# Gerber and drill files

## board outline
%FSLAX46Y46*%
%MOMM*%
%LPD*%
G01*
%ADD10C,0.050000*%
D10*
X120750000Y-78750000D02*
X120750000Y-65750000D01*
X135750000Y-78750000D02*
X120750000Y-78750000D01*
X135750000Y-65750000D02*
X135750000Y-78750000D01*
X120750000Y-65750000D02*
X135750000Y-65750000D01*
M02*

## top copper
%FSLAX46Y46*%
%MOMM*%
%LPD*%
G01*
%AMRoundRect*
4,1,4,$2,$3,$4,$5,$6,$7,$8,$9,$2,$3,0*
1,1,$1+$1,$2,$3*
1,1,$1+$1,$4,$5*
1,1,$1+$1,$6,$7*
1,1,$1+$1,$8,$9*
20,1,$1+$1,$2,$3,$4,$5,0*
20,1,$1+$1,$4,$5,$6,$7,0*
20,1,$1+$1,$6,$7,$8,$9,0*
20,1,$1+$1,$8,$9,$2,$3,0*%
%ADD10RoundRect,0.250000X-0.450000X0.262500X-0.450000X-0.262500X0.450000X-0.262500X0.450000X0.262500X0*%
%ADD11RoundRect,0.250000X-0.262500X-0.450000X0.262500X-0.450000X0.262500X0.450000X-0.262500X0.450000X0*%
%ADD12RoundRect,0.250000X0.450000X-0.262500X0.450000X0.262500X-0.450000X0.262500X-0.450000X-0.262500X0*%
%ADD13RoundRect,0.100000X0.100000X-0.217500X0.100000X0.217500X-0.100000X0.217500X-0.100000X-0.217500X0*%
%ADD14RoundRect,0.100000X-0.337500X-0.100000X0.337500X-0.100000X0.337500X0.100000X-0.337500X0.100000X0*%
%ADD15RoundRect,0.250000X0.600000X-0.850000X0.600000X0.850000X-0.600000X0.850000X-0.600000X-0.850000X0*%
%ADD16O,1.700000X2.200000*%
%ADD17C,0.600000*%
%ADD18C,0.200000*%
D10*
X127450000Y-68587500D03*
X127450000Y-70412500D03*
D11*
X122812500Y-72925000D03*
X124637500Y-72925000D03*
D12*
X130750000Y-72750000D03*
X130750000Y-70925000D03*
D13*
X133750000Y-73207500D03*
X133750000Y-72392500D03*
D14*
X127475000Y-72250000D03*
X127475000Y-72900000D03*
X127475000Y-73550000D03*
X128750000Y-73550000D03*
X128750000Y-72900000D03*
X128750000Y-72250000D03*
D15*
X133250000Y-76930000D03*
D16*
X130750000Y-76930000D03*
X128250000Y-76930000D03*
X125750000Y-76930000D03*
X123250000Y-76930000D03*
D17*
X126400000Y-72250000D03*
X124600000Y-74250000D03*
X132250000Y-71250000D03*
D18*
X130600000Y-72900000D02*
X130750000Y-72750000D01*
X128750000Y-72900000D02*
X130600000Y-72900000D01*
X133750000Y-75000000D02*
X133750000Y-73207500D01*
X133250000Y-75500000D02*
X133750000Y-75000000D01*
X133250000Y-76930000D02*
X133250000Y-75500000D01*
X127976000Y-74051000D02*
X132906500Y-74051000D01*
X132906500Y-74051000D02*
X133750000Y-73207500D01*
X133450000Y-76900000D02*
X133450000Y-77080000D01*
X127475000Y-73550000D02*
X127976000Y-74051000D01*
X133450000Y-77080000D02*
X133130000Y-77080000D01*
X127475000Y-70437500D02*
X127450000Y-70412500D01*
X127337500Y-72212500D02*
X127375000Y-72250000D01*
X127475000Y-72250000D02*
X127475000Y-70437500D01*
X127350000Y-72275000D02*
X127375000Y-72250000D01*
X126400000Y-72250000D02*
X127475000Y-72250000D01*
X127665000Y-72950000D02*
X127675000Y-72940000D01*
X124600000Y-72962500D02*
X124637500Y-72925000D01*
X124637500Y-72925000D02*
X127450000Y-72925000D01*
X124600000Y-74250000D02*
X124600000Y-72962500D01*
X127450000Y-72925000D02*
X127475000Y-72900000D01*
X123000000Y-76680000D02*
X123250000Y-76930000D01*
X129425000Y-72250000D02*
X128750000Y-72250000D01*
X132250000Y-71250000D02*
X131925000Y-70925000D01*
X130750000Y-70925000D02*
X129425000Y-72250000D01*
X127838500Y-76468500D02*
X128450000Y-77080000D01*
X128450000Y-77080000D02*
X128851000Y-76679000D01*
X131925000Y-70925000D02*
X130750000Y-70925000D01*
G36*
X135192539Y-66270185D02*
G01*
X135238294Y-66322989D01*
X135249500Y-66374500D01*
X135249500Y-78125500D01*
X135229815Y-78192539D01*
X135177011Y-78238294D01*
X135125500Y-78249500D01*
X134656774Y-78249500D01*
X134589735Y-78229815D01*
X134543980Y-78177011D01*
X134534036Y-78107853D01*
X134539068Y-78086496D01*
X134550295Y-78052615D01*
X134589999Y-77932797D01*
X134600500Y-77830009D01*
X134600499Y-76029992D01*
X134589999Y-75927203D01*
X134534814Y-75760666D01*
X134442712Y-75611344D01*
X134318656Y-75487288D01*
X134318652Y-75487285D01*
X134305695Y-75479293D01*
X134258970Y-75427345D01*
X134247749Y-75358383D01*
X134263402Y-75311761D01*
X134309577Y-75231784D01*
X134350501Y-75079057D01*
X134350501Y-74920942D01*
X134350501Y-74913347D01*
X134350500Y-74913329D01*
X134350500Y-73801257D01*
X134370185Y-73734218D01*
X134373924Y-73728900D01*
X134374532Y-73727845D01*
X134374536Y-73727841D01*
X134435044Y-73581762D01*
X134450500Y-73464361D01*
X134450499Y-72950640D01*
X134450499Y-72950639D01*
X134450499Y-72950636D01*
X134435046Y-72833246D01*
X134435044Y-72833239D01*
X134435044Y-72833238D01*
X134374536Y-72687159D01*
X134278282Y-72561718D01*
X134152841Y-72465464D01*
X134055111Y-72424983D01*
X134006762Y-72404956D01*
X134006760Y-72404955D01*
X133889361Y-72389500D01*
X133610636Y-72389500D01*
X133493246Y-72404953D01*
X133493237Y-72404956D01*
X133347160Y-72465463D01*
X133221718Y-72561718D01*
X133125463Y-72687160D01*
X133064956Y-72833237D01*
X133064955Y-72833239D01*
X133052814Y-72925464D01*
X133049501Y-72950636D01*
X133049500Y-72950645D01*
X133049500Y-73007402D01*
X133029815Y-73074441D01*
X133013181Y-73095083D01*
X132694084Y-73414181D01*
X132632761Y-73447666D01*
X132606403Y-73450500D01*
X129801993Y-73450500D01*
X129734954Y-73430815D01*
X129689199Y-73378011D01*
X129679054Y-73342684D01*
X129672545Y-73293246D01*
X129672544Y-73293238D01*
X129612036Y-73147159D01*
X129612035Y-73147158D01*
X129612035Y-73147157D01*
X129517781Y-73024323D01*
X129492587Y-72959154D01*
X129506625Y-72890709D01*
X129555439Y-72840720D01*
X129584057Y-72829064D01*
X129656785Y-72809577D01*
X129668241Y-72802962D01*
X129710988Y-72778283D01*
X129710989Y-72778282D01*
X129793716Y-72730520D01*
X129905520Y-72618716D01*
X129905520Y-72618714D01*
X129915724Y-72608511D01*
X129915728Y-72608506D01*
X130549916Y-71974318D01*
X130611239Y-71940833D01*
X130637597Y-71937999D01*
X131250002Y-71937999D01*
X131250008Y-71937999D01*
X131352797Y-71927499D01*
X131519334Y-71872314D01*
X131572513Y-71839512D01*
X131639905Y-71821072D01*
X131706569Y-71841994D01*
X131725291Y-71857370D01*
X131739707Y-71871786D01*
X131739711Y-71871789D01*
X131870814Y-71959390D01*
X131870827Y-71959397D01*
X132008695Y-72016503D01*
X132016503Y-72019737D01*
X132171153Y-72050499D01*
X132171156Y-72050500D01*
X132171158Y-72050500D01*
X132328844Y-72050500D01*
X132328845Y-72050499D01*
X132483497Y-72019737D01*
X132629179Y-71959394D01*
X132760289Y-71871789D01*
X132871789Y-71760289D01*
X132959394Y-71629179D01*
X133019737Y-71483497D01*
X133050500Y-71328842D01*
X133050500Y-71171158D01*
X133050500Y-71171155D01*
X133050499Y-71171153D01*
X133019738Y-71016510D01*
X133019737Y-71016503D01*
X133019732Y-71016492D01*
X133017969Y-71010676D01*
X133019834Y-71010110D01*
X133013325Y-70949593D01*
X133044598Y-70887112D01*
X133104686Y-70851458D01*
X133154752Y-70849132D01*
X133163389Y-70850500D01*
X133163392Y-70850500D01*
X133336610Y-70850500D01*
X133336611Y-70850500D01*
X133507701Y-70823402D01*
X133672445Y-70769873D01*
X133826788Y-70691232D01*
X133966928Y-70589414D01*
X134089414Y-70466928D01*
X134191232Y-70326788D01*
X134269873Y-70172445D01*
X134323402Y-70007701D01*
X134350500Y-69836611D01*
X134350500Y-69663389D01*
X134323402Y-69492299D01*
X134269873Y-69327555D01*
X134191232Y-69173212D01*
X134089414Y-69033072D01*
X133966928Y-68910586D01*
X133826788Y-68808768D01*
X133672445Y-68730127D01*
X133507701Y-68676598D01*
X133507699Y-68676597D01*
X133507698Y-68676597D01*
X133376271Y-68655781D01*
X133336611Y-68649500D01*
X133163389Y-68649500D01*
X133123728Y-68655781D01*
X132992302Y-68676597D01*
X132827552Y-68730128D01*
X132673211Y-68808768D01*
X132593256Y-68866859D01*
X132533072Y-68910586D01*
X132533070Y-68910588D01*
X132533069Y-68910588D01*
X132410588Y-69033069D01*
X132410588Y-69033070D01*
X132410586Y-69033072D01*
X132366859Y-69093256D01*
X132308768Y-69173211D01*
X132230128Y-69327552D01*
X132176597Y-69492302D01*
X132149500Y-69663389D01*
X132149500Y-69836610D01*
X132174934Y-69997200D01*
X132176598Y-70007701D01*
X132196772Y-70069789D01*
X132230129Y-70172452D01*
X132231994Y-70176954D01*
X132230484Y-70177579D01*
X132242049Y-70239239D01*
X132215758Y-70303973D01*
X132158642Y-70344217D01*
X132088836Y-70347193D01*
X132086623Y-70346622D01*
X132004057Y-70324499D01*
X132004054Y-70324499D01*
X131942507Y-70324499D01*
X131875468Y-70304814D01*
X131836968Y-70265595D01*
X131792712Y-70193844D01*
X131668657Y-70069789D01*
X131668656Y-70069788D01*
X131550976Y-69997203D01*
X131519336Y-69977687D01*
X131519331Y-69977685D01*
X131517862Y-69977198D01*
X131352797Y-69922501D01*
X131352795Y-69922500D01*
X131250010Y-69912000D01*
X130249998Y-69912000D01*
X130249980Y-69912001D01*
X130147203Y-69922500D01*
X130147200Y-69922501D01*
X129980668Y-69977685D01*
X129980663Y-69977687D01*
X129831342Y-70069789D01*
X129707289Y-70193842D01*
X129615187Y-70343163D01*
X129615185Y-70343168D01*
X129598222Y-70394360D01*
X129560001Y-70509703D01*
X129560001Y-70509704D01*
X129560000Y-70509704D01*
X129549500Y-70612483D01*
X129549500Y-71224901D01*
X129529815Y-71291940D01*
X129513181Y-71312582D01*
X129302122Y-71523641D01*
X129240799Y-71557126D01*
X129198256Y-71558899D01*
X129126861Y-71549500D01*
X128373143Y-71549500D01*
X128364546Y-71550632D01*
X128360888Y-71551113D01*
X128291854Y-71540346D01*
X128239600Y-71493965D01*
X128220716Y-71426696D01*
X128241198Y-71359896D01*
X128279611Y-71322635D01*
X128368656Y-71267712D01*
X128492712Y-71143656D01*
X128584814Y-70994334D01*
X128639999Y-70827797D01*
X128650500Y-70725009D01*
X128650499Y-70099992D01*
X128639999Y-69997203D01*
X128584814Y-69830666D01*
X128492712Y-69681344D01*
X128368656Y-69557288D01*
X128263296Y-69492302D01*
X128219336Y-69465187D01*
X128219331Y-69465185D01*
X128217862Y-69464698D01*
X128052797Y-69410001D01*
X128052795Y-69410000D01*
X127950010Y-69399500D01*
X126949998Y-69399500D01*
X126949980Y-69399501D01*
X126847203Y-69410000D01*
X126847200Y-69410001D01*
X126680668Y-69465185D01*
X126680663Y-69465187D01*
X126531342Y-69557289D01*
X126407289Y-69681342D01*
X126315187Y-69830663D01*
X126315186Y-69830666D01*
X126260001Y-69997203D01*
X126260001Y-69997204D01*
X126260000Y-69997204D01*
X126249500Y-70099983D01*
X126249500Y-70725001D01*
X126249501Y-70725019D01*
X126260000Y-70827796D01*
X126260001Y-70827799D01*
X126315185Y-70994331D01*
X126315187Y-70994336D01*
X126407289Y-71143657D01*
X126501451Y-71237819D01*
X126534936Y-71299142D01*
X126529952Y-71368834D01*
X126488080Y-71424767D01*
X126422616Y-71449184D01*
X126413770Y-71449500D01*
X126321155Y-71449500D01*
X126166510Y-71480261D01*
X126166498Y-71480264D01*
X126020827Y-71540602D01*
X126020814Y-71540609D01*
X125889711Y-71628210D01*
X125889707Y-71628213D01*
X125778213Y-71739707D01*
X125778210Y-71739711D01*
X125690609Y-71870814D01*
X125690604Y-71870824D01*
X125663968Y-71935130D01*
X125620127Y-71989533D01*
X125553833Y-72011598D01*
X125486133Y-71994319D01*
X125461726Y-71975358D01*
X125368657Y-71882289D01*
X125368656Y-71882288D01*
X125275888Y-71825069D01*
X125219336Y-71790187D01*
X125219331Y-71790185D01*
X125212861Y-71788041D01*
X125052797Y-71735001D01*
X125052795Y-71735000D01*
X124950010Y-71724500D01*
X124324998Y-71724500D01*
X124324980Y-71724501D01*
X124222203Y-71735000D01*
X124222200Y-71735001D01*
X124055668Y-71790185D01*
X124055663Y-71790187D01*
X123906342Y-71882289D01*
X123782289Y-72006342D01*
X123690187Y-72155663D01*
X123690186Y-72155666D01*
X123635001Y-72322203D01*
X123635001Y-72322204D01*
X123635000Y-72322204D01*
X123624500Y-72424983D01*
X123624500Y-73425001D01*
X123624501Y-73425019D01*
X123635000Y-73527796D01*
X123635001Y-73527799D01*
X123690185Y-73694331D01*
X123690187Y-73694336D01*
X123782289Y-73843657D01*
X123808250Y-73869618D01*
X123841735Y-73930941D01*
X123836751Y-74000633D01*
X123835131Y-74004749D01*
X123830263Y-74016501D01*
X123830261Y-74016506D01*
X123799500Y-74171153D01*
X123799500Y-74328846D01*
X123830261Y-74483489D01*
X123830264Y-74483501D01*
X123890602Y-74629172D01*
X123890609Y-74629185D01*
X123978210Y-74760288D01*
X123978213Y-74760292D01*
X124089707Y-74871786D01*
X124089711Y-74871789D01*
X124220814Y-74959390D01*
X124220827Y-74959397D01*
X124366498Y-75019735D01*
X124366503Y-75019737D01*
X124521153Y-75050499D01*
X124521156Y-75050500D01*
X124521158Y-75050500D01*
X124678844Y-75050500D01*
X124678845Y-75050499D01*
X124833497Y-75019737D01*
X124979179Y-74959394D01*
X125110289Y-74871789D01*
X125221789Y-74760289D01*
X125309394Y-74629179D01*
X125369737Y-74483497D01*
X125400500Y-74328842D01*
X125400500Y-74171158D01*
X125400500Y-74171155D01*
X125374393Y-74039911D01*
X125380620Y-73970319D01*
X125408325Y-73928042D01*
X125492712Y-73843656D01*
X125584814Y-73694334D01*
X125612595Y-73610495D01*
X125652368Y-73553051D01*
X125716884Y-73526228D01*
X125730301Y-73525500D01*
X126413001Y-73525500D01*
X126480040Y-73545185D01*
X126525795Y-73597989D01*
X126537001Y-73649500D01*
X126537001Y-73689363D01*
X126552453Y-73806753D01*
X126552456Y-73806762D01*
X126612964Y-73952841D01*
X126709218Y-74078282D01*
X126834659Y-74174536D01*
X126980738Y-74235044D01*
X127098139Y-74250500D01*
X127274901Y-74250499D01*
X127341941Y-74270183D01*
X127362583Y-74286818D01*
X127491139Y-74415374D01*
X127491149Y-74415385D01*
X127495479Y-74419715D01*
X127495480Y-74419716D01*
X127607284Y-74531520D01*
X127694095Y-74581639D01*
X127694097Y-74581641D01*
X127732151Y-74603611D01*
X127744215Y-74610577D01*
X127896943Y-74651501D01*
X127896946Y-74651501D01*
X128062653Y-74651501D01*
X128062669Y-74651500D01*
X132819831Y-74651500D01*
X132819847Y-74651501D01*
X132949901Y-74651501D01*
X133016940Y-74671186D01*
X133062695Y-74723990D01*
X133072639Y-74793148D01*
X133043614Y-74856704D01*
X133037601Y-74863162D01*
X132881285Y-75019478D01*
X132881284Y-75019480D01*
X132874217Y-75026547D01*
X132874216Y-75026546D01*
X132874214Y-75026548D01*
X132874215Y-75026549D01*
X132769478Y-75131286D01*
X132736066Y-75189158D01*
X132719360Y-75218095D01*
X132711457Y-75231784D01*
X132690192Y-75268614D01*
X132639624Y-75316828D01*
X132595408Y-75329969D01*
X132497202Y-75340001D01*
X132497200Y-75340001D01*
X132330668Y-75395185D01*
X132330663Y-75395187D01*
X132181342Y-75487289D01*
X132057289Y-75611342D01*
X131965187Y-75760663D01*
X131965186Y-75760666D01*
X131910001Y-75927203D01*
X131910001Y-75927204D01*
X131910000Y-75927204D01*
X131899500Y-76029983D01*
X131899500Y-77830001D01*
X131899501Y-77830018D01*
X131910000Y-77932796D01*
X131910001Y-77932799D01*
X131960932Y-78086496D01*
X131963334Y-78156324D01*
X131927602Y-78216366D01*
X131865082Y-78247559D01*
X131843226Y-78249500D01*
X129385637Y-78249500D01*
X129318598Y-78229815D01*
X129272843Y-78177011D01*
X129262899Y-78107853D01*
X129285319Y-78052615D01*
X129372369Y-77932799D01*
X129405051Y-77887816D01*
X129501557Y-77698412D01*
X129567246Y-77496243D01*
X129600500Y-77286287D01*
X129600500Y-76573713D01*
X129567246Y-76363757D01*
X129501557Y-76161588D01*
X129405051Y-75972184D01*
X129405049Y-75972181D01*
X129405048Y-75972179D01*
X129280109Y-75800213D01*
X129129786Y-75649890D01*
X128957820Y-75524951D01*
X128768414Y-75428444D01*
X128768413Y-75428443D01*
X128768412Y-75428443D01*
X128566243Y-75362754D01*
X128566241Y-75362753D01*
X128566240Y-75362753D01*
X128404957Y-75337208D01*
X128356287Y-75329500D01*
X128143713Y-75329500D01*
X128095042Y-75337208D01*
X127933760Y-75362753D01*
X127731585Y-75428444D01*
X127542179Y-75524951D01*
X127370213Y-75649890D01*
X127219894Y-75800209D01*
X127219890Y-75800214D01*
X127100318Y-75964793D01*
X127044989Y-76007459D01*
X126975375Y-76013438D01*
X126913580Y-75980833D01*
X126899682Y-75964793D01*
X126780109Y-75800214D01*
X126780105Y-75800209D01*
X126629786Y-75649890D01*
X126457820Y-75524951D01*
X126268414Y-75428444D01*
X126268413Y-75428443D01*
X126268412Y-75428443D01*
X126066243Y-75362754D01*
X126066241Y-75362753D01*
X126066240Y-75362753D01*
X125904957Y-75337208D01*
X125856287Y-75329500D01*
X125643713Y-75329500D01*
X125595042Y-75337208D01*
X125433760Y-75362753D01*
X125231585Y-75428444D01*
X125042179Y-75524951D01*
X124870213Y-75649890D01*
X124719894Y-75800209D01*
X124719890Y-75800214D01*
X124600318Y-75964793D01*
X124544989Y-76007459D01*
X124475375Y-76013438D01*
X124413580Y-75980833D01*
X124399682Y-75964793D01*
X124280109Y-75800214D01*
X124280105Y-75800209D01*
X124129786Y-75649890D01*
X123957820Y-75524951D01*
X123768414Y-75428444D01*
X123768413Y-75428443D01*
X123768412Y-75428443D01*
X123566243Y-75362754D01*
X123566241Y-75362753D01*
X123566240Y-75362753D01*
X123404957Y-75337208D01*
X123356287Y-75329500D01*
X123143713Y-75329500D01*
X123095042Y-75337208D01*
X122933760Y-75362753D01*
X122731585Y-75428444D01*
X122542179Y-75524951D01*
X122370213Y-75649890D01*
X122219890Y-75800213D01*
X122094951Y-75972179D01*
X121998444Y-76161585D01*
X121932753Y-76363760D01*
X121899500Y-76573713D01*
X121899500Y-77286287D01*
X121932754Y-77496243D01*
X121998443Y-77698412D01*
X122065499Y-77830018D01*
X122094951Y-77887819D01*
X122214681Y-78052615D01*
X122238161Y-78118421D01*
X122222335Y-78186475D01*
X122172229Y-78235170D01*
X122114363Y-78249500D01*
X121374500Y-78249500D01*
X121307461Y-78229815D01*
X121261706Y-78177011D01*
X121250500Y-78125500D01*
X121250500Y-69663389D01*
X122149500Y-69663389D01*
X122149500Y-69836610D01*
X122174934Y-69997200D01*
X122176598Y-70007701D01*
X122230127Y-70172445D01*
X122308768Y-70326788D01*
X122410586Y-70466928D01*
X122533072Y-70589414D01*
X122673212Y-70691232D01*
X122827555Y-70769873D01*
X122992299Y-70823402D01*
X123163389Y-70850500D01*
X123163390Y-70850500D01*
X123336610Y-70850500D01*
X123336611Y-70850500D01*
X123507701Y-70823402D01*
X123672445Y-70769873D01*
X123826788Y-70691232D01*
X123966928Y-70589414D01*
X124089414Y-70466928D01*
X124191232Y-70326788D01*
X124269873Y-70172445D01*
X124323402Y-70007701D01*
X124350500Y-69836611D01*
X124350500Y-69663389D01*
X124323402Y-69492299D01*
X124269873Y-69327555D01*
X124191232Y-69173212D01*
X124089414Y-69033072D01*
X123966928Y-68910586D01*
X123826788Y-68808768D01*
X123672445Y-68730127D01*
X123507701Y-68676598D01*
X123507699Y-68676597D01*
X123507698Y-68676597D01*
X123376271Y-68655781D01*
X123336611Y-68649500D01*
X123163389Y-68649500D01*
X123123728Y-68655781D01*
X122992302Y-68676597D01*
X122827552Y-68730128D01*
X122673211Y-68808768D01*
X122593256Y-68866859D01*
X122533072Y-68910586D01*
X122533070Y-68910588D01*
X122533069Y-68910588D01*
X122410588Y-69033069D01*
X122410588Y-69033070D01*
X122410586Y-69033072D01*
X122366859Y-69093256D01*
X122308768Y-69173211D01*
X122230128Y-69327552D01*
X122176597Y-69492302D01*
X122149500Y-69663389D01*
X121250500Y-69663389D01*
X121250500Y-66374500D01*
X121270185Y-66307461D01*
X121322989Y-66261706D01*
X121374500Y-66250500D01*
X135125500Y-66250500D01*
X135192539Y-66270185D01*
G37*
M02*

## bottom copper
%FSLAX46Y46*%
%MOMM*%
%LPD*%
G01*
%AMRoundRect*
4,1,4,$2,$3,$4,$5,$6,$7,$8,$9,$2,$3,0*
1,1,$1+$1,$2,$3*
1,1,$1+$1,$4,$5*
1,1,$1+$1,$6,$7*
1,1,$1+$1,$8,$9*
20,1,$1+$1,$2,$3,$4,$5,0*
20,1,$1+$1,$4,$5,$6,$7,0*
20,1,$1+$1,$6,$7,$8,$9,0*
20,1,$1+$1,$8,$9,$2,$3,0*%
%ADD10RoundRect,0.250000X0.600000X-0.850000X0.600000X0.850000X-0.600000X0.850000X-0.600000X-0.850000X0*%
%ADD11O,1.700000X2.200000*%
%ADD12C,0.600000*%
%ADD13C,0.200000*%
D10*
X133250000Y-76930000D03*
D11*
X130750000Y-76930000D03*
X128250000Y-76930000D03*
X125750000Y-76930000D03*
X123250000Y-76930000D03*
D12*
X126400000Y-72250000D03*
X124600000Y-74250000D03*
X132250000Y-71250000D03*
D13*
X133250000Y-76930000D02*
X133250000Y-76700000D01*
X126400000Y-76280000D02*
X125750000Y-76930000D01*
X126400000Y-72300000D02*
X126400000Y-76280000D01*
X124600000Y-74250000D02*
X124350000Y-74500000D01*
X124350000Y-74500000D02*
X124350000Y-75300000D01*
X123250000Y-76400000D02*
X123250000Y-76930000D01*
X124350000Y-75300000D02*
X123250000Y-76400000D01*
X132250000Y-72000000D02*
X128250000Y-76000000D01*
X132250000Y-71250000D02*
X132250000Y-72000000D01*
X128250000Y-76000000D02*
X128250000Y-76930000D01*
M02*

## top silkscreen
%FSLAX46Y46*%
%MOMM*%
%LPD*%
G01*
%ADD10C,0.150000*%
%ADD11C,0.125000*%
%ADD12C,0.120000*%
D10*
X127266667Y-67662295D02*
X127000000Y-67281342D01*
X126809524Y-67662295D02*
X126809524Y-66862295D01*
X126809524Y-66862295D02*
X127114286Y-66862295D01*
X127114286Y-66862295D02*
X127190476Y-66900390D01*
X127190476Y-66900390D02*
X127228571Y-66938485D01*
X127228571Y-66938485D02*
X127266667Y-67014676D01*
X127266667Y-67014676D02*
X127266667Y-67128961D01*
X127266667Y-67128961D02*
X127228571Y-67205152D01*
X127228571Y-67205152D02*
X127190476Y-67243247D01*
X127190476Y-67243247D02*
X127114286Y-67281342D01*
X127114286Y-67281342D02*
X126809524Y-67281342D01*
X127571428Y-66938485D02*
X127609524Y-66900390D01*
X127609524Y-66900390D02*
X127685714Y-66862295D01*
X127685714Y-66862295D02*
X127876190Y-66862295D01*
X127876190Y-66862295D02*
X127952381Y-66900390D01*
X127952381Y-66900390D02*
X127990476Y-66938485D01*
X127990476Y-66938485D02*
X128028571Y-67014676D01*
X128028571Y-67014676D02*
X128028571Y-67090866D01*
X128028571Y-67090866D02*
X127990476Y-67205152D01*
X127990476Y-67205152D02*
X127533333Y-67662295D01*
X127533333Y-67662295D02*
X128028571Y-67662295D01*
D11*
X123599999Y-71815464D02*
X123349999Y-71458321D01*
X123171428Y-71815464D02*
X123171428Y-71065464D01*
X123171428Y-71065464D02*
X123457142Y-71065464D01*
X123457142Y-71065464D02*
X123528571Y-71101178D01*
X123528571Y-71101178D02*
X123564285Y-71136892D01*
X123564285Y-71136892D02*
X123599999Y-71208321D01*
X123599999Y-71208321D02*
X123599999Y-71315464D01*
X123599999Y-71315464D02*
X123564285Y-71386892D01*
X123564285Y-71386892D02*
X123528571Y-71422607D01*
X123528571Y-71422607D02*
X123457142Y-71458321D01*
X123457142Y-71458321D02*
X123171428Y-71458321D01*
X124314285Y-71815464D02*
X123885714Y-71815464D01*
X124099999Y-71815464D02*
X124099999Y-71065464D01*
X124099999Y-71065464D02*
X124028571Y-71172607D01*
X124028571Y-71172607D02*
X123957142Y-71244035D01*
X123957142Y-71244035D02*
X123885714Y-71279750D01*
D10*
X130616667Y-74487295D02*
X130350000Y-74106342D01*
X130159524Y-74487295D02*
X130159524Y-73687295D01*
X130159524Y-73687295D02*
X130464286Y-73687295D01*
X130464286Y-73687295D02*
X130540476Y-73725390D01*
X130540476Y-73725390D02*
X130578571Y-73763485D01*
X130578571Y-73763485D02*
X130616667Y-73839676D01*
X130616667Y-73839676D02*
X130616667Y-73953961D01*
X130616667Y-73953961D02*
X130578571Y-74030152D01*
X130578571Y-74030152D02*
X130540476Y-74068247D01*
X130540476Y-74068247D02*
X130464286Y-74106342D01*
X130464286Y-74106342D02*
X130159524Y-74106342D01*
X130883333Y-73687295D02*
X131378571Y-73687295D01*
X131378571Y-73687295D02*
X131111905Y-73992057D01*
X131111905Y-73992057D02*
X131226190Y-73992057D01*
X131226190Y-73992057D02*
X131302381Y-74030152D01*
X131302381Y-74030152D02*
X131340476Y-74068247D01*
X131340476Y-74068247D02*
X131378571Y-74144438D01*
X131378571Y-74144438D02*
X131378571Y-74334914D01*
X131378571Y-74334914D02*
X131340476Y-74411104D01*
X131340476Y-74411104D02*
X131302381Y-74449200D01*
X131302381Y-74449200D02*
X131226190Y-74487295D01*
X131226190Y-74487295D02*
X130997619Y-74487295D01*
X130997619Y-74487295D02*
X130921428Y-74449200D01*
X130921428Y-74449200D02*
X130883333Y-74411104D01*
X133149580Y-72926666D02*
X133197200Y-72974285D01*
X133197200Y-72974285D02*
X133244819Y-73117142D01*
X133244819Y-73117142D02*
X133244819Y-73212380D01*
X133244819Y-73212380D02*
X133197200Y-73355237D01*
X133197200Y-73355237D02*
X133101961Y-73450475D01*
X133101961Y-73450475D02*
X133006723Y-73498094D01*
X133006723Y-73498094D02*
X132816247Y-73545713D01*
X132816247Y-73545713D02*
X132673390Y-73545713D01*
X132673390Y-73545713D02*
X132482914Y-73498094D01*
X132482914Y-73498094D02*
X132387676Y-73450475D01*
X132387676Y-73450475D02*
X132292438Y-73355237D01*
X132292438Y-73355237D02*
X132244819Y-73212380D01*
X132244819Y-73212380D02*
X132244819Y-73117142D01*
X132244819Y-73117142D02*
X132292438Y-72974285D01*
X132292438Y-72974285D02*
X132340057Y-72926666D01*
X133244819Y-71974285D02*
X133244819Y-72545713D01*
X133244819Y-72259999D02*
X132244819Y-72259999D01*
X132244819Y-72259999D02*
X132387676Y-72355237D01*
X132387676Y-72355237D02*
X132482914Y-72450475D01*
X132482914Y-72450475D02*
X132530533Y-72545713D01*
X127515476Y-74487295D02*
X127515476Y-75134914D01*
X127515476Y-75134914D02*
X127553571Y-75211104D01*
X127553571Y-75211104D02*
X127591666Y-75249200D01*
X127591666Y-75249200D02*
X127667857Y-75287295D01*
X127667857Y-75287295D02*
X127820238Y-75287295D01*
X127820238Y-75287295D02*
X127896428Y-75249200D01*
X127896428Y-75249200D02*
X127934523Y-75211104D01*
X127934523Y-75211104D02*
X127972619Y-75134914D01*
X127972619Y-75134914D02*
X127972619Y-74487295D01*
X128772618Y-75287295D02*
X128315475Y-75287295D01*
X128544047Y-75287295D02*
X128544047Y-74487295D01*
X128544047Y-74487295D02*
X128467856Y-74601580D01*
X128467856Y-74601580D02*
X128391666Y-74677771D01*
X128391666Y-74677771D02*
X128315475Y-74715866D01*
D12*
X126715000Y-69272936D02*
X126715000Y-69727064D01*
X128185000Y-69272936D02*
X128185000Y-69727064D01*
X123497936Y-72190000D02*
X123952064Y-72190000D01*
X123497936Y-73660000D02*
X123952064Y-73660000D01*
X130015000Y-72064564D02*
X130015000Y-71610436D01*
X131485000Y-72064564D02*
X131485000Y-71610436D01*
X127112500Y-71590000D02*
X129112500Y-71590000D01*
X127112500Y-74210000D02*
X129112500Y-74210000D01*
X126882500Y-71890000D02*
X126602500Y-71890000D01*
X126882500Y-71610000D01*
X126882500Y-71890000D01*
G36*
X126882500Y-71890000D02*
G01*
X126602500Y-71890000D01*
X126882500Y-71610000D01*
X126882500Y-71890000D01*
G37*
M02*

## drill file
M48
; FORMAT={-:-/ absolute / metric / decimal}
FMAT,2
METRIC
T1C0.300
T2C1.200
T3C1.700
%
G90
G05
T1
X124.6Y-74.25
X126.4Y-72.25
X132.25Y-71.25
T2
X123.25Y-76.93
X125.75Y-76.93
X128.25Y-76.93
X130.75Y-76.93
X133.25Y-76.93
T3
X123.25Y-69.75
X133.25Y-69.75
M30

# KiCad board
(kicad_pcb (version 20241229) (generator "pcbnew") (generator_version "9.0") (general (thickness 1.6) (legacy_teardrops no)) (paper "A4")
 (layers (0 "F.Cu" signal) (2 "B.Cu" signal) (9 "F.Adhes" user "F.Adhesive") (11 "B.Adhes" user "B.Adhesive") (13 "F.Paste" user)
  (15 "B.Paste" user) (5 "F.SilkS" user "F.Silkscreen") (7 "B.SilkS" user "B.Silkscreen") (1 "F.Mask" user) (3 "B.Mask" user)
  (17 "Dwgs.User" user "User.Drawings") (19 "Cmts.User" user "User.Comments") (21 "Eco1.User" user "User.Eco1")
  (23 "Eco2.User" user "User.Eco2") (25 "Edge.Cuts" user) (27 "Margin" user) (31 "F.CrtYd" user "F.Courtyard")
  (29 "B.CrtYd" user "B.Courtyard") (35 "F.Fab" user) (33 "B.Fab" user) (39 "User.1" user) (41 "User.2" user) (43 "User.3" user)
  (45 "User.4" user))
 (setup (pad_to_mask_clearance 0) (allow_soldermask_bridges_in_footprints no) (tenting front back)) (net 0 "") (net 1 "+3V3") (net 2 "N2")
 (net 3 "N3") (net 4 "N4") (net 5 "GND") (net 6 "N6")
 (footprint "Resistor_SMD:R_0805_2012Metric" (layer "F.Cu") (at 127.45 69.5 -90)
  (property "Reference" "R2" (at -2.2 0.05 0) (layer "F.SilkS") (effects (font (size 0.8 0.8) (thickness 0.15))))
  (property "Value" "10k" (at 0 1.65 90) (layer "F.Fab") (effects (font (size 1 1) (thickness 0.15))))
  (fp_line (start -0.227064 0.735) (end 0.227064 0.735) (stroke (width 0.12) (type solid)) (layer "F.SilkS"))
  (fp_line (start -0.227064 -0.735) (end 0.227064 -0.735) (stroke (width 0.12) (type solid)) (layer "F.SilkS"))
  (pad "1" smd roundrect (at -0.9125 0 270) (size 1.025 1.4) (layers "F.Cu" "F.Mask" "F.Paste") (roundrect_rratio 0.243902) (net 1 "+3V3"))
  (pad "2" smd roundrect (at 0.9125 0 270) (size 1.025 1.4) (layers "F.Cu" "F.Mask" "F.Paste") (roundrect_rratio 0.243902) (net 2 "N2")))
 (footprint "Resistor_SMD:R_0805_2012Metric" (layer "F.Cu") (at 123.725 72.925)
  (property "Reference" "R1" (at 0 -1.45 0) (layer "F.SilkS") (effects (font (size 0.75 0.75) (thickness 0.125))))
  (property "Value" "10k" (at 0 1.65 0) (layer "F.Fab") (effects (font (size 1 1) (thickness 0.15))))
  (fp_line (start -0.227064 -0.735) (end 0.227064 -0.735) (stroke (width 0.12) (type solid)) (layer "F.SilkS"))
  (fp_line (start -0.227064 0.735) (end 0.227064 0.735) (stroke (width 0.12) (type solid)) (layer "F.SilkS"))
  (pad "1" smd roundrect (at -0.9125 0) (size 1.025 1.4) (layers "F.Cu" "F.Mask" "F.Paste") (roundrect_rratio 0.243902) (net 1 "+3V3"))
  (pad "2" smd roundrect (at 0.9125 0) (size 1.025 1.4) (layers "F.Cu" "F.Mask" "F.Paste") (roundrect_rratio 0.243902) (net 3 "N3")))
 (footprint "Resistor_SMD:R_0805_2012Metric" (layer "F.Cu") (at 130.75 71.8375 90)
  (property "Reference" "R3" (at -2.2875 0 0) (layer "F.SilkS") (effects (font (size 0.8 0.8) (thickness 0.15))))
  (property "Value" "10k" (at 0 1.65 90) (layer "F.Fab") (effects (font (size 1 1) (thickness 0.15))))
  (fp_line (start -0.227064 -0.735) (end 0.227064 -0.735) (stroke (width 0.12) (type solid)) (layer "F.SilkS"))
  (fp_line (start -0.227064 0.735) (end 0.227064 0.735) (stroke (width 0.12) (type solid)) (layer "F.SilkS"))
  (pad "1" smd roundrect (at -0.9125 0 90) (size 1.025 1.4) (layers "F.Cu" "F.Mask" "F.Paste") (roundrect_rratio 0.243902) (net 1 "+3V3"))
  (pad "2" smd roundrect (at 0.9125 0 90) (size 1.025 1.4) (layers "F.Cu" "F.Mask" "F.Paste") (roundrect_rratio 0.243902) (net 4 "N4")))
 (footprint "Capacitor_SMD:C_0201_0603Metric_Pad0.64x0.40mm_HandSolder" (layer "F.Cu") (at 133.75 72.8 90)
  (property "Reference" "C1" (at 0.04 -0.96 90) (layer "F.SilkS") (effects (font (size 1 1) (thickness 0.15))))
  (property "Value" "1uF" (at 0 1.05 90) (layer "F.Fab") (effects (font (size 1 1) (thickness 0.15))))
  (pad "" smd roundrect (at -0.4325 0 90) (size 0.458 0.36) (layers "F.Paste") (roundrect_rratio 0.25))
  (pad "" smd roundrect (at 0.4325 0 90) (size 0.458 0.36) (layers "F.Paste") (roundrect_rratio 0.25))
  (pad "1" smd roundrect (at -0.4075 0 90) (size 0.635 0.4) (layers "F.Cu" "F.Mask") (roundrect_rratio 0.25) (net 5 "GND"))
  (pad "2" smd roundrect (at 0.4075 0 90) (size 0.635 0.4) (layers "F.Cu" "F.Mask") (roundrect_rratio 0.25) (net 1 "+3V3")))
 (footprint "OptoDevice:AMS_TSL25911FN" (layer "F.Cu") (at 128.1125 72.9)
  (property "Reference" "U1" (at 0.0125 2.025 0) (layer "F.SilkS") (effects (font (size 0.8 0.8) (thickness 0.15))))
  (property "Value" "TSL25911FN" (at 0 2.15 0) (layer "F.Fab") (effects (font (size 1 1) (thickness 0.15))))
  (fp_line (start -1 -1.31) (end 1 -1.31) (stroke (width 0.12) (type solid)) (layer "F.SilkS"))
  (fp_line (start -1 1.31) (end 1 1.31) (stroke (width 0.12) (type solid)) (layer "F.SilkS"))
  (fp_poly
   (pts (xy -1.23 -1.01) (xy -1.51 -1.01) (xy -1.23 -1.29) (xy -1.23 -1.01)) (stroke (width 0.12) (type solid)) (fill yes) (layer "F.SilkS"))
  (pad "1" smd roundrect (at -0.6375 -0.65) (size 0.875 0.4) (layers "F.Cu" "F.Mask" "F.Paste") (roundrect_rratio 0.25) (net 2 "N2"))
  (pad "2" smd roundrect (at -0.6375 0) (size 0.875 0.4) (layers "F.Cu" "F.Mask" "F.Paste") (roundrect_rratio 0.25) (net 3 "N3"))
  (pad "3" smd roundrect (at -0.6375 0.65) (size 0.875 0.4) (layers "F.Cu" "F.Mask" "F.Paste") (roundrect_rratio 0.25) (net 5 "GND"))
  (pad "4" smd roundrect (at 0.6375 0.65) (size 0.875 0.4) (layers "F.Cu" "F.Mask" "F.Paste") (roundrect_rratio 0.25) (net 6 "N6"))
  (pad "5" smd roundrect (at 0.6375 0) (size 0.875 0.4) (layers "F.Cu" "F.Mask" "F.Paste") (roundrect_rratio 0.25) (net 1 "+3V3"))
  (pad "6" smd roundrect (at 0.6375 -0.65) (size 0.875 0.4) (layers "F.Cu" "F.Mask" "F.Paste") (roundrect_rratio 0.25) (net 4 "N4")))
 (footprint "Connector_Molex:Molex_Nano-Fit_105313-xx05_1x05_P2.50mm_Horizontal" (layer "B.Cu") (at 133.25 76.93 90)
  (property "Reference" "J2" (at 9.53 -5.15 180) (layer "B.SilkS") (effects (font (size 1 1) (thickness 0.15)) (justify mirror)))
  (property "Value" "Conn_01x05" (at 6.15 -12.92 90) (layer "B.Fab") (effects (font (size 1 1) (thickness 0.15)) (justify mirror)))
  (pad "" np_thru_hole circle (at 7.18 -10 90) (size 1.7 1.7) (drill 1.7) (layers "*.Cu" "*.Mask"))
  (pad "" np_thru_hole circle (at 7.18 0 90) (size 1.7 1.7) (drill 1.7) (layers "*.Cu" "*.Mask"))
  (pad "1" thru_hole roundrect (at 0 0 90) (size 2.2 1.7) (drill 1.2) (layers "*.Cu" "*.Mask") (remove_unused_layers no)
   (roundrect_rratio 0.147059) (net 5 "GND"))
  (pad "2" thru_hole oval (at 0 -2.5 90) (size 2.2 1.7) (drill 1.2) (layers "*.Cu" "*.Mask") (remove_unused_layers no) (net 1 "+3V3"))
  (pad "3" thru_hole oval (at 0 -5 90) (size 2.2 1.7) (drill 1.2) (layers "*.Cu" "*.Mask") (remove_unused_layers no) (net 4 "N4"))
  (pad "4" thru_hole oval (at 0 -7.5 90) (size 2.2 1.7) (drill 1.2) (layers "*.Cu" "*.Mask") (remove_unused_layers no) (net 2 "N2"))
  (pad "5" thru_hole oval (at 0 -10 90) (size 2.2 1.7) (drill 1.2) (layers "*.Cu" "*.Mask") (remove_unused_layers no) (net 3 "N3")))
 (gr_line (start 120.75 78.75) (end 120.75 65.75) (stroke (width 0.05) (type default)) (layer "Edge.Cuts"))
 (gr_line (start 135.75 78.75) (end 120.75 78.75) (stroke (width 0.05) (type default)) (layer "Edge.Cuts"))
 (gr_line (start 135.75 65.75) (end 135.75 78.75) (stroke (width 0.05) (type default)) (layer "Edge.Cuts"))
 (gr_line (start 120.75 65.75) (end 135.75 65.75) (stroke (width 0.05) (type default)) (layer "Edge.Cuts"))
 (segment (start 130.6 72.9) (end 130.75 72.75) (width 0.2) (layer "F.Cu") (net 1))
 (segment (start 128.75 72.9) (end 130.6 72.9) (width 0.2) (layer "F.Cu") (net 1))
 (segment (start 133.75 75) (end 133.75 73.2075) (width 0.2) (layer "F.Cu") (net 5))
 (segment (start 133.25 75.5) (end 133.75 75) (width 0.2) (layer "F.Cu") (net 5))
 (segment (start 133.25 76.93) (end 133.25 75.5) (width 0.2) (layer "F.Cu") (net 5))
 (segment (start 127.976 74.051) (end 132.9065 74.051) (width 0.2) (layer "F.Cu") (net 5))
 (segment (start 132.9065 74.051) (end 133.75 73.2075) (width 0.2) (layer "F.Cu") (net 5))
 (segment (start 133.45 76.9) (end 133.45 77.08) (width 0.2) (layer "F.Cu") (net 5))
 (segment (start 127.475 73.55) (end 127.976 74.051) (width 0.2) (layer "F.Cu") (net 5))
 (segment (start 133.45 77.08) (end 133.13 77.08) (width 0.2) (layer "F.Cu") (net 5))
 (segment (start 133.25 76.93) (end 133.25 76.7) (width 0.2) (layer "B.Cu") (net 5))
 (segment (start 127.475 70.4375) (end 127.45 70.4125) (width 0.2) (layer "F.Cu") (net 2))
 (segment (start 127.3375 72.2125) (end 127.375 72.25) (width 0.2) (layer "F.Cu") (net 2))
 (segment (start 127.475 72.25) (end 127.475 70.4375) (width 0.2) (layer "F.Cu") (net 2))
 (segment (start 127.35 72.275) (end 127.375 72.25) (width 0.2) (layer "F.Cu") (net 2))
 (segment (start 126.4 72.25) (end 127.475 72.25) (width 0.2) (layer "F.Cu") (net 2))
 (via (at 126.4 72.25) (size 0.6) (drill 0.3) (layers "F.Cu" "B.Cu") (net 2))
 (segment (start 126.4 76.28) (end 125.75 76.93) (width 0.2) (layer "B.Cu") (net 2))
 (segment (start 126.4 72.3) (end 126.4 76.28) (width 0.2) (layer "B.Cu") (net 2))
 (segment (start 127.665 72.95) (end 127.675 72.94) (width 0.2) (layer "F.Cu") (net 3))
 (segment (start 124.6 72.9625) (end 124.6375 72.925) (width 0.2) (layer "F.Cu") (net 3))
 (segment (start 124.6375 72.925) (end 127.45 72.925) (width 0.2) (layer "F.Cu") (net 3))
 (segment (start 124.6 74.25) (end 124.6 72.9625) (width 0.2) (layer "F.Cu") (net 3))
 (segment (start 127.45 72.925) (end 127.475 72.9) (width 0.2) (layer "F.Cu") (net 3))
 (segment (start 123 76.68) (end 123.25 76.93) (width 0.2) (layer "F.Cu") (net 3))
 (via (at 124.6 74.25) (size 0.6) (drill 0.3) (layers "F.Cu" "B.Cu") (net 3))
 (segment (start 124.6 74.25) (end 124.35 74.5) (width 0.2) (layer "B.Cu") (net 3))
 (segment (start 124.35 74.5) (end 124.35 75.3) (width 0.2) (layer "B.Cu") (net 3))
 (segment (start 123.25 76.4) (end 123.25 76.93) (width 0.2) (layer "B.Cu") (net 3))
 (segment (start 124.35 75.3) (end 123.25 76.4) (width 0.2) (layer "B.Cu") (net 3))
 (segment (start 129.425 72.25) (end 128.75 72.25) (width 0.2) (layer "F.Cu") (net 4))
 (segment (start 132.25 71.25) (end 131.925 70.925) (width 0.2) (layer "F.Cu") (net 4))
 (segment (start 130.75 70.925) (end 129.425 72.25) (width 0.2) (layer "F.Cu") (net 4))
 (segment (start 127.8385 76.4685) (end 128.45 77.08) (width 0.2) (layer "F.Cu") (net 4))
 (segment (start 128.45 77.08) (end 128.851 76.679) (width 0.2) (layer "F.Cu") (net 4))
 (segment (start 131.925 70.925) (end 130.75 70.925) (width 0.2) (layer "F.Cu") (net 4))
 (via (at 132.25 71.25) (size 0.6) (drill 0.3) (layers "F.Cu" "B.Cu") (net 4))
 (segment (start 132.25 72) (end 128.25 76) (width 0.2) (layer "B.Cu") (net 4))
 (segment (start 132.25 71.25) (end 132.25 72) (width 0.2) (layer "B.Cu") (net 4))
 (segment (start 128.25 76) (end 128.25 76.93) (width 0.2) (layer "B.Cu") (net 4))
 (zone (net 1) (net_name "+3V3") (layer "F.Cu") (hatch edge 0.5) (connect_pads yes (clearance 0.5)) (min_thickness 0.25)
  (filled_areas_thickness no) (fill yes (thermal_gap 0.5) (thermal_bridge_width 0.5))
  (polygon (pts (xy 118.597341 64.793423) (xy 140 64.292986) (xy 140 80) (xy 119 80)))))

